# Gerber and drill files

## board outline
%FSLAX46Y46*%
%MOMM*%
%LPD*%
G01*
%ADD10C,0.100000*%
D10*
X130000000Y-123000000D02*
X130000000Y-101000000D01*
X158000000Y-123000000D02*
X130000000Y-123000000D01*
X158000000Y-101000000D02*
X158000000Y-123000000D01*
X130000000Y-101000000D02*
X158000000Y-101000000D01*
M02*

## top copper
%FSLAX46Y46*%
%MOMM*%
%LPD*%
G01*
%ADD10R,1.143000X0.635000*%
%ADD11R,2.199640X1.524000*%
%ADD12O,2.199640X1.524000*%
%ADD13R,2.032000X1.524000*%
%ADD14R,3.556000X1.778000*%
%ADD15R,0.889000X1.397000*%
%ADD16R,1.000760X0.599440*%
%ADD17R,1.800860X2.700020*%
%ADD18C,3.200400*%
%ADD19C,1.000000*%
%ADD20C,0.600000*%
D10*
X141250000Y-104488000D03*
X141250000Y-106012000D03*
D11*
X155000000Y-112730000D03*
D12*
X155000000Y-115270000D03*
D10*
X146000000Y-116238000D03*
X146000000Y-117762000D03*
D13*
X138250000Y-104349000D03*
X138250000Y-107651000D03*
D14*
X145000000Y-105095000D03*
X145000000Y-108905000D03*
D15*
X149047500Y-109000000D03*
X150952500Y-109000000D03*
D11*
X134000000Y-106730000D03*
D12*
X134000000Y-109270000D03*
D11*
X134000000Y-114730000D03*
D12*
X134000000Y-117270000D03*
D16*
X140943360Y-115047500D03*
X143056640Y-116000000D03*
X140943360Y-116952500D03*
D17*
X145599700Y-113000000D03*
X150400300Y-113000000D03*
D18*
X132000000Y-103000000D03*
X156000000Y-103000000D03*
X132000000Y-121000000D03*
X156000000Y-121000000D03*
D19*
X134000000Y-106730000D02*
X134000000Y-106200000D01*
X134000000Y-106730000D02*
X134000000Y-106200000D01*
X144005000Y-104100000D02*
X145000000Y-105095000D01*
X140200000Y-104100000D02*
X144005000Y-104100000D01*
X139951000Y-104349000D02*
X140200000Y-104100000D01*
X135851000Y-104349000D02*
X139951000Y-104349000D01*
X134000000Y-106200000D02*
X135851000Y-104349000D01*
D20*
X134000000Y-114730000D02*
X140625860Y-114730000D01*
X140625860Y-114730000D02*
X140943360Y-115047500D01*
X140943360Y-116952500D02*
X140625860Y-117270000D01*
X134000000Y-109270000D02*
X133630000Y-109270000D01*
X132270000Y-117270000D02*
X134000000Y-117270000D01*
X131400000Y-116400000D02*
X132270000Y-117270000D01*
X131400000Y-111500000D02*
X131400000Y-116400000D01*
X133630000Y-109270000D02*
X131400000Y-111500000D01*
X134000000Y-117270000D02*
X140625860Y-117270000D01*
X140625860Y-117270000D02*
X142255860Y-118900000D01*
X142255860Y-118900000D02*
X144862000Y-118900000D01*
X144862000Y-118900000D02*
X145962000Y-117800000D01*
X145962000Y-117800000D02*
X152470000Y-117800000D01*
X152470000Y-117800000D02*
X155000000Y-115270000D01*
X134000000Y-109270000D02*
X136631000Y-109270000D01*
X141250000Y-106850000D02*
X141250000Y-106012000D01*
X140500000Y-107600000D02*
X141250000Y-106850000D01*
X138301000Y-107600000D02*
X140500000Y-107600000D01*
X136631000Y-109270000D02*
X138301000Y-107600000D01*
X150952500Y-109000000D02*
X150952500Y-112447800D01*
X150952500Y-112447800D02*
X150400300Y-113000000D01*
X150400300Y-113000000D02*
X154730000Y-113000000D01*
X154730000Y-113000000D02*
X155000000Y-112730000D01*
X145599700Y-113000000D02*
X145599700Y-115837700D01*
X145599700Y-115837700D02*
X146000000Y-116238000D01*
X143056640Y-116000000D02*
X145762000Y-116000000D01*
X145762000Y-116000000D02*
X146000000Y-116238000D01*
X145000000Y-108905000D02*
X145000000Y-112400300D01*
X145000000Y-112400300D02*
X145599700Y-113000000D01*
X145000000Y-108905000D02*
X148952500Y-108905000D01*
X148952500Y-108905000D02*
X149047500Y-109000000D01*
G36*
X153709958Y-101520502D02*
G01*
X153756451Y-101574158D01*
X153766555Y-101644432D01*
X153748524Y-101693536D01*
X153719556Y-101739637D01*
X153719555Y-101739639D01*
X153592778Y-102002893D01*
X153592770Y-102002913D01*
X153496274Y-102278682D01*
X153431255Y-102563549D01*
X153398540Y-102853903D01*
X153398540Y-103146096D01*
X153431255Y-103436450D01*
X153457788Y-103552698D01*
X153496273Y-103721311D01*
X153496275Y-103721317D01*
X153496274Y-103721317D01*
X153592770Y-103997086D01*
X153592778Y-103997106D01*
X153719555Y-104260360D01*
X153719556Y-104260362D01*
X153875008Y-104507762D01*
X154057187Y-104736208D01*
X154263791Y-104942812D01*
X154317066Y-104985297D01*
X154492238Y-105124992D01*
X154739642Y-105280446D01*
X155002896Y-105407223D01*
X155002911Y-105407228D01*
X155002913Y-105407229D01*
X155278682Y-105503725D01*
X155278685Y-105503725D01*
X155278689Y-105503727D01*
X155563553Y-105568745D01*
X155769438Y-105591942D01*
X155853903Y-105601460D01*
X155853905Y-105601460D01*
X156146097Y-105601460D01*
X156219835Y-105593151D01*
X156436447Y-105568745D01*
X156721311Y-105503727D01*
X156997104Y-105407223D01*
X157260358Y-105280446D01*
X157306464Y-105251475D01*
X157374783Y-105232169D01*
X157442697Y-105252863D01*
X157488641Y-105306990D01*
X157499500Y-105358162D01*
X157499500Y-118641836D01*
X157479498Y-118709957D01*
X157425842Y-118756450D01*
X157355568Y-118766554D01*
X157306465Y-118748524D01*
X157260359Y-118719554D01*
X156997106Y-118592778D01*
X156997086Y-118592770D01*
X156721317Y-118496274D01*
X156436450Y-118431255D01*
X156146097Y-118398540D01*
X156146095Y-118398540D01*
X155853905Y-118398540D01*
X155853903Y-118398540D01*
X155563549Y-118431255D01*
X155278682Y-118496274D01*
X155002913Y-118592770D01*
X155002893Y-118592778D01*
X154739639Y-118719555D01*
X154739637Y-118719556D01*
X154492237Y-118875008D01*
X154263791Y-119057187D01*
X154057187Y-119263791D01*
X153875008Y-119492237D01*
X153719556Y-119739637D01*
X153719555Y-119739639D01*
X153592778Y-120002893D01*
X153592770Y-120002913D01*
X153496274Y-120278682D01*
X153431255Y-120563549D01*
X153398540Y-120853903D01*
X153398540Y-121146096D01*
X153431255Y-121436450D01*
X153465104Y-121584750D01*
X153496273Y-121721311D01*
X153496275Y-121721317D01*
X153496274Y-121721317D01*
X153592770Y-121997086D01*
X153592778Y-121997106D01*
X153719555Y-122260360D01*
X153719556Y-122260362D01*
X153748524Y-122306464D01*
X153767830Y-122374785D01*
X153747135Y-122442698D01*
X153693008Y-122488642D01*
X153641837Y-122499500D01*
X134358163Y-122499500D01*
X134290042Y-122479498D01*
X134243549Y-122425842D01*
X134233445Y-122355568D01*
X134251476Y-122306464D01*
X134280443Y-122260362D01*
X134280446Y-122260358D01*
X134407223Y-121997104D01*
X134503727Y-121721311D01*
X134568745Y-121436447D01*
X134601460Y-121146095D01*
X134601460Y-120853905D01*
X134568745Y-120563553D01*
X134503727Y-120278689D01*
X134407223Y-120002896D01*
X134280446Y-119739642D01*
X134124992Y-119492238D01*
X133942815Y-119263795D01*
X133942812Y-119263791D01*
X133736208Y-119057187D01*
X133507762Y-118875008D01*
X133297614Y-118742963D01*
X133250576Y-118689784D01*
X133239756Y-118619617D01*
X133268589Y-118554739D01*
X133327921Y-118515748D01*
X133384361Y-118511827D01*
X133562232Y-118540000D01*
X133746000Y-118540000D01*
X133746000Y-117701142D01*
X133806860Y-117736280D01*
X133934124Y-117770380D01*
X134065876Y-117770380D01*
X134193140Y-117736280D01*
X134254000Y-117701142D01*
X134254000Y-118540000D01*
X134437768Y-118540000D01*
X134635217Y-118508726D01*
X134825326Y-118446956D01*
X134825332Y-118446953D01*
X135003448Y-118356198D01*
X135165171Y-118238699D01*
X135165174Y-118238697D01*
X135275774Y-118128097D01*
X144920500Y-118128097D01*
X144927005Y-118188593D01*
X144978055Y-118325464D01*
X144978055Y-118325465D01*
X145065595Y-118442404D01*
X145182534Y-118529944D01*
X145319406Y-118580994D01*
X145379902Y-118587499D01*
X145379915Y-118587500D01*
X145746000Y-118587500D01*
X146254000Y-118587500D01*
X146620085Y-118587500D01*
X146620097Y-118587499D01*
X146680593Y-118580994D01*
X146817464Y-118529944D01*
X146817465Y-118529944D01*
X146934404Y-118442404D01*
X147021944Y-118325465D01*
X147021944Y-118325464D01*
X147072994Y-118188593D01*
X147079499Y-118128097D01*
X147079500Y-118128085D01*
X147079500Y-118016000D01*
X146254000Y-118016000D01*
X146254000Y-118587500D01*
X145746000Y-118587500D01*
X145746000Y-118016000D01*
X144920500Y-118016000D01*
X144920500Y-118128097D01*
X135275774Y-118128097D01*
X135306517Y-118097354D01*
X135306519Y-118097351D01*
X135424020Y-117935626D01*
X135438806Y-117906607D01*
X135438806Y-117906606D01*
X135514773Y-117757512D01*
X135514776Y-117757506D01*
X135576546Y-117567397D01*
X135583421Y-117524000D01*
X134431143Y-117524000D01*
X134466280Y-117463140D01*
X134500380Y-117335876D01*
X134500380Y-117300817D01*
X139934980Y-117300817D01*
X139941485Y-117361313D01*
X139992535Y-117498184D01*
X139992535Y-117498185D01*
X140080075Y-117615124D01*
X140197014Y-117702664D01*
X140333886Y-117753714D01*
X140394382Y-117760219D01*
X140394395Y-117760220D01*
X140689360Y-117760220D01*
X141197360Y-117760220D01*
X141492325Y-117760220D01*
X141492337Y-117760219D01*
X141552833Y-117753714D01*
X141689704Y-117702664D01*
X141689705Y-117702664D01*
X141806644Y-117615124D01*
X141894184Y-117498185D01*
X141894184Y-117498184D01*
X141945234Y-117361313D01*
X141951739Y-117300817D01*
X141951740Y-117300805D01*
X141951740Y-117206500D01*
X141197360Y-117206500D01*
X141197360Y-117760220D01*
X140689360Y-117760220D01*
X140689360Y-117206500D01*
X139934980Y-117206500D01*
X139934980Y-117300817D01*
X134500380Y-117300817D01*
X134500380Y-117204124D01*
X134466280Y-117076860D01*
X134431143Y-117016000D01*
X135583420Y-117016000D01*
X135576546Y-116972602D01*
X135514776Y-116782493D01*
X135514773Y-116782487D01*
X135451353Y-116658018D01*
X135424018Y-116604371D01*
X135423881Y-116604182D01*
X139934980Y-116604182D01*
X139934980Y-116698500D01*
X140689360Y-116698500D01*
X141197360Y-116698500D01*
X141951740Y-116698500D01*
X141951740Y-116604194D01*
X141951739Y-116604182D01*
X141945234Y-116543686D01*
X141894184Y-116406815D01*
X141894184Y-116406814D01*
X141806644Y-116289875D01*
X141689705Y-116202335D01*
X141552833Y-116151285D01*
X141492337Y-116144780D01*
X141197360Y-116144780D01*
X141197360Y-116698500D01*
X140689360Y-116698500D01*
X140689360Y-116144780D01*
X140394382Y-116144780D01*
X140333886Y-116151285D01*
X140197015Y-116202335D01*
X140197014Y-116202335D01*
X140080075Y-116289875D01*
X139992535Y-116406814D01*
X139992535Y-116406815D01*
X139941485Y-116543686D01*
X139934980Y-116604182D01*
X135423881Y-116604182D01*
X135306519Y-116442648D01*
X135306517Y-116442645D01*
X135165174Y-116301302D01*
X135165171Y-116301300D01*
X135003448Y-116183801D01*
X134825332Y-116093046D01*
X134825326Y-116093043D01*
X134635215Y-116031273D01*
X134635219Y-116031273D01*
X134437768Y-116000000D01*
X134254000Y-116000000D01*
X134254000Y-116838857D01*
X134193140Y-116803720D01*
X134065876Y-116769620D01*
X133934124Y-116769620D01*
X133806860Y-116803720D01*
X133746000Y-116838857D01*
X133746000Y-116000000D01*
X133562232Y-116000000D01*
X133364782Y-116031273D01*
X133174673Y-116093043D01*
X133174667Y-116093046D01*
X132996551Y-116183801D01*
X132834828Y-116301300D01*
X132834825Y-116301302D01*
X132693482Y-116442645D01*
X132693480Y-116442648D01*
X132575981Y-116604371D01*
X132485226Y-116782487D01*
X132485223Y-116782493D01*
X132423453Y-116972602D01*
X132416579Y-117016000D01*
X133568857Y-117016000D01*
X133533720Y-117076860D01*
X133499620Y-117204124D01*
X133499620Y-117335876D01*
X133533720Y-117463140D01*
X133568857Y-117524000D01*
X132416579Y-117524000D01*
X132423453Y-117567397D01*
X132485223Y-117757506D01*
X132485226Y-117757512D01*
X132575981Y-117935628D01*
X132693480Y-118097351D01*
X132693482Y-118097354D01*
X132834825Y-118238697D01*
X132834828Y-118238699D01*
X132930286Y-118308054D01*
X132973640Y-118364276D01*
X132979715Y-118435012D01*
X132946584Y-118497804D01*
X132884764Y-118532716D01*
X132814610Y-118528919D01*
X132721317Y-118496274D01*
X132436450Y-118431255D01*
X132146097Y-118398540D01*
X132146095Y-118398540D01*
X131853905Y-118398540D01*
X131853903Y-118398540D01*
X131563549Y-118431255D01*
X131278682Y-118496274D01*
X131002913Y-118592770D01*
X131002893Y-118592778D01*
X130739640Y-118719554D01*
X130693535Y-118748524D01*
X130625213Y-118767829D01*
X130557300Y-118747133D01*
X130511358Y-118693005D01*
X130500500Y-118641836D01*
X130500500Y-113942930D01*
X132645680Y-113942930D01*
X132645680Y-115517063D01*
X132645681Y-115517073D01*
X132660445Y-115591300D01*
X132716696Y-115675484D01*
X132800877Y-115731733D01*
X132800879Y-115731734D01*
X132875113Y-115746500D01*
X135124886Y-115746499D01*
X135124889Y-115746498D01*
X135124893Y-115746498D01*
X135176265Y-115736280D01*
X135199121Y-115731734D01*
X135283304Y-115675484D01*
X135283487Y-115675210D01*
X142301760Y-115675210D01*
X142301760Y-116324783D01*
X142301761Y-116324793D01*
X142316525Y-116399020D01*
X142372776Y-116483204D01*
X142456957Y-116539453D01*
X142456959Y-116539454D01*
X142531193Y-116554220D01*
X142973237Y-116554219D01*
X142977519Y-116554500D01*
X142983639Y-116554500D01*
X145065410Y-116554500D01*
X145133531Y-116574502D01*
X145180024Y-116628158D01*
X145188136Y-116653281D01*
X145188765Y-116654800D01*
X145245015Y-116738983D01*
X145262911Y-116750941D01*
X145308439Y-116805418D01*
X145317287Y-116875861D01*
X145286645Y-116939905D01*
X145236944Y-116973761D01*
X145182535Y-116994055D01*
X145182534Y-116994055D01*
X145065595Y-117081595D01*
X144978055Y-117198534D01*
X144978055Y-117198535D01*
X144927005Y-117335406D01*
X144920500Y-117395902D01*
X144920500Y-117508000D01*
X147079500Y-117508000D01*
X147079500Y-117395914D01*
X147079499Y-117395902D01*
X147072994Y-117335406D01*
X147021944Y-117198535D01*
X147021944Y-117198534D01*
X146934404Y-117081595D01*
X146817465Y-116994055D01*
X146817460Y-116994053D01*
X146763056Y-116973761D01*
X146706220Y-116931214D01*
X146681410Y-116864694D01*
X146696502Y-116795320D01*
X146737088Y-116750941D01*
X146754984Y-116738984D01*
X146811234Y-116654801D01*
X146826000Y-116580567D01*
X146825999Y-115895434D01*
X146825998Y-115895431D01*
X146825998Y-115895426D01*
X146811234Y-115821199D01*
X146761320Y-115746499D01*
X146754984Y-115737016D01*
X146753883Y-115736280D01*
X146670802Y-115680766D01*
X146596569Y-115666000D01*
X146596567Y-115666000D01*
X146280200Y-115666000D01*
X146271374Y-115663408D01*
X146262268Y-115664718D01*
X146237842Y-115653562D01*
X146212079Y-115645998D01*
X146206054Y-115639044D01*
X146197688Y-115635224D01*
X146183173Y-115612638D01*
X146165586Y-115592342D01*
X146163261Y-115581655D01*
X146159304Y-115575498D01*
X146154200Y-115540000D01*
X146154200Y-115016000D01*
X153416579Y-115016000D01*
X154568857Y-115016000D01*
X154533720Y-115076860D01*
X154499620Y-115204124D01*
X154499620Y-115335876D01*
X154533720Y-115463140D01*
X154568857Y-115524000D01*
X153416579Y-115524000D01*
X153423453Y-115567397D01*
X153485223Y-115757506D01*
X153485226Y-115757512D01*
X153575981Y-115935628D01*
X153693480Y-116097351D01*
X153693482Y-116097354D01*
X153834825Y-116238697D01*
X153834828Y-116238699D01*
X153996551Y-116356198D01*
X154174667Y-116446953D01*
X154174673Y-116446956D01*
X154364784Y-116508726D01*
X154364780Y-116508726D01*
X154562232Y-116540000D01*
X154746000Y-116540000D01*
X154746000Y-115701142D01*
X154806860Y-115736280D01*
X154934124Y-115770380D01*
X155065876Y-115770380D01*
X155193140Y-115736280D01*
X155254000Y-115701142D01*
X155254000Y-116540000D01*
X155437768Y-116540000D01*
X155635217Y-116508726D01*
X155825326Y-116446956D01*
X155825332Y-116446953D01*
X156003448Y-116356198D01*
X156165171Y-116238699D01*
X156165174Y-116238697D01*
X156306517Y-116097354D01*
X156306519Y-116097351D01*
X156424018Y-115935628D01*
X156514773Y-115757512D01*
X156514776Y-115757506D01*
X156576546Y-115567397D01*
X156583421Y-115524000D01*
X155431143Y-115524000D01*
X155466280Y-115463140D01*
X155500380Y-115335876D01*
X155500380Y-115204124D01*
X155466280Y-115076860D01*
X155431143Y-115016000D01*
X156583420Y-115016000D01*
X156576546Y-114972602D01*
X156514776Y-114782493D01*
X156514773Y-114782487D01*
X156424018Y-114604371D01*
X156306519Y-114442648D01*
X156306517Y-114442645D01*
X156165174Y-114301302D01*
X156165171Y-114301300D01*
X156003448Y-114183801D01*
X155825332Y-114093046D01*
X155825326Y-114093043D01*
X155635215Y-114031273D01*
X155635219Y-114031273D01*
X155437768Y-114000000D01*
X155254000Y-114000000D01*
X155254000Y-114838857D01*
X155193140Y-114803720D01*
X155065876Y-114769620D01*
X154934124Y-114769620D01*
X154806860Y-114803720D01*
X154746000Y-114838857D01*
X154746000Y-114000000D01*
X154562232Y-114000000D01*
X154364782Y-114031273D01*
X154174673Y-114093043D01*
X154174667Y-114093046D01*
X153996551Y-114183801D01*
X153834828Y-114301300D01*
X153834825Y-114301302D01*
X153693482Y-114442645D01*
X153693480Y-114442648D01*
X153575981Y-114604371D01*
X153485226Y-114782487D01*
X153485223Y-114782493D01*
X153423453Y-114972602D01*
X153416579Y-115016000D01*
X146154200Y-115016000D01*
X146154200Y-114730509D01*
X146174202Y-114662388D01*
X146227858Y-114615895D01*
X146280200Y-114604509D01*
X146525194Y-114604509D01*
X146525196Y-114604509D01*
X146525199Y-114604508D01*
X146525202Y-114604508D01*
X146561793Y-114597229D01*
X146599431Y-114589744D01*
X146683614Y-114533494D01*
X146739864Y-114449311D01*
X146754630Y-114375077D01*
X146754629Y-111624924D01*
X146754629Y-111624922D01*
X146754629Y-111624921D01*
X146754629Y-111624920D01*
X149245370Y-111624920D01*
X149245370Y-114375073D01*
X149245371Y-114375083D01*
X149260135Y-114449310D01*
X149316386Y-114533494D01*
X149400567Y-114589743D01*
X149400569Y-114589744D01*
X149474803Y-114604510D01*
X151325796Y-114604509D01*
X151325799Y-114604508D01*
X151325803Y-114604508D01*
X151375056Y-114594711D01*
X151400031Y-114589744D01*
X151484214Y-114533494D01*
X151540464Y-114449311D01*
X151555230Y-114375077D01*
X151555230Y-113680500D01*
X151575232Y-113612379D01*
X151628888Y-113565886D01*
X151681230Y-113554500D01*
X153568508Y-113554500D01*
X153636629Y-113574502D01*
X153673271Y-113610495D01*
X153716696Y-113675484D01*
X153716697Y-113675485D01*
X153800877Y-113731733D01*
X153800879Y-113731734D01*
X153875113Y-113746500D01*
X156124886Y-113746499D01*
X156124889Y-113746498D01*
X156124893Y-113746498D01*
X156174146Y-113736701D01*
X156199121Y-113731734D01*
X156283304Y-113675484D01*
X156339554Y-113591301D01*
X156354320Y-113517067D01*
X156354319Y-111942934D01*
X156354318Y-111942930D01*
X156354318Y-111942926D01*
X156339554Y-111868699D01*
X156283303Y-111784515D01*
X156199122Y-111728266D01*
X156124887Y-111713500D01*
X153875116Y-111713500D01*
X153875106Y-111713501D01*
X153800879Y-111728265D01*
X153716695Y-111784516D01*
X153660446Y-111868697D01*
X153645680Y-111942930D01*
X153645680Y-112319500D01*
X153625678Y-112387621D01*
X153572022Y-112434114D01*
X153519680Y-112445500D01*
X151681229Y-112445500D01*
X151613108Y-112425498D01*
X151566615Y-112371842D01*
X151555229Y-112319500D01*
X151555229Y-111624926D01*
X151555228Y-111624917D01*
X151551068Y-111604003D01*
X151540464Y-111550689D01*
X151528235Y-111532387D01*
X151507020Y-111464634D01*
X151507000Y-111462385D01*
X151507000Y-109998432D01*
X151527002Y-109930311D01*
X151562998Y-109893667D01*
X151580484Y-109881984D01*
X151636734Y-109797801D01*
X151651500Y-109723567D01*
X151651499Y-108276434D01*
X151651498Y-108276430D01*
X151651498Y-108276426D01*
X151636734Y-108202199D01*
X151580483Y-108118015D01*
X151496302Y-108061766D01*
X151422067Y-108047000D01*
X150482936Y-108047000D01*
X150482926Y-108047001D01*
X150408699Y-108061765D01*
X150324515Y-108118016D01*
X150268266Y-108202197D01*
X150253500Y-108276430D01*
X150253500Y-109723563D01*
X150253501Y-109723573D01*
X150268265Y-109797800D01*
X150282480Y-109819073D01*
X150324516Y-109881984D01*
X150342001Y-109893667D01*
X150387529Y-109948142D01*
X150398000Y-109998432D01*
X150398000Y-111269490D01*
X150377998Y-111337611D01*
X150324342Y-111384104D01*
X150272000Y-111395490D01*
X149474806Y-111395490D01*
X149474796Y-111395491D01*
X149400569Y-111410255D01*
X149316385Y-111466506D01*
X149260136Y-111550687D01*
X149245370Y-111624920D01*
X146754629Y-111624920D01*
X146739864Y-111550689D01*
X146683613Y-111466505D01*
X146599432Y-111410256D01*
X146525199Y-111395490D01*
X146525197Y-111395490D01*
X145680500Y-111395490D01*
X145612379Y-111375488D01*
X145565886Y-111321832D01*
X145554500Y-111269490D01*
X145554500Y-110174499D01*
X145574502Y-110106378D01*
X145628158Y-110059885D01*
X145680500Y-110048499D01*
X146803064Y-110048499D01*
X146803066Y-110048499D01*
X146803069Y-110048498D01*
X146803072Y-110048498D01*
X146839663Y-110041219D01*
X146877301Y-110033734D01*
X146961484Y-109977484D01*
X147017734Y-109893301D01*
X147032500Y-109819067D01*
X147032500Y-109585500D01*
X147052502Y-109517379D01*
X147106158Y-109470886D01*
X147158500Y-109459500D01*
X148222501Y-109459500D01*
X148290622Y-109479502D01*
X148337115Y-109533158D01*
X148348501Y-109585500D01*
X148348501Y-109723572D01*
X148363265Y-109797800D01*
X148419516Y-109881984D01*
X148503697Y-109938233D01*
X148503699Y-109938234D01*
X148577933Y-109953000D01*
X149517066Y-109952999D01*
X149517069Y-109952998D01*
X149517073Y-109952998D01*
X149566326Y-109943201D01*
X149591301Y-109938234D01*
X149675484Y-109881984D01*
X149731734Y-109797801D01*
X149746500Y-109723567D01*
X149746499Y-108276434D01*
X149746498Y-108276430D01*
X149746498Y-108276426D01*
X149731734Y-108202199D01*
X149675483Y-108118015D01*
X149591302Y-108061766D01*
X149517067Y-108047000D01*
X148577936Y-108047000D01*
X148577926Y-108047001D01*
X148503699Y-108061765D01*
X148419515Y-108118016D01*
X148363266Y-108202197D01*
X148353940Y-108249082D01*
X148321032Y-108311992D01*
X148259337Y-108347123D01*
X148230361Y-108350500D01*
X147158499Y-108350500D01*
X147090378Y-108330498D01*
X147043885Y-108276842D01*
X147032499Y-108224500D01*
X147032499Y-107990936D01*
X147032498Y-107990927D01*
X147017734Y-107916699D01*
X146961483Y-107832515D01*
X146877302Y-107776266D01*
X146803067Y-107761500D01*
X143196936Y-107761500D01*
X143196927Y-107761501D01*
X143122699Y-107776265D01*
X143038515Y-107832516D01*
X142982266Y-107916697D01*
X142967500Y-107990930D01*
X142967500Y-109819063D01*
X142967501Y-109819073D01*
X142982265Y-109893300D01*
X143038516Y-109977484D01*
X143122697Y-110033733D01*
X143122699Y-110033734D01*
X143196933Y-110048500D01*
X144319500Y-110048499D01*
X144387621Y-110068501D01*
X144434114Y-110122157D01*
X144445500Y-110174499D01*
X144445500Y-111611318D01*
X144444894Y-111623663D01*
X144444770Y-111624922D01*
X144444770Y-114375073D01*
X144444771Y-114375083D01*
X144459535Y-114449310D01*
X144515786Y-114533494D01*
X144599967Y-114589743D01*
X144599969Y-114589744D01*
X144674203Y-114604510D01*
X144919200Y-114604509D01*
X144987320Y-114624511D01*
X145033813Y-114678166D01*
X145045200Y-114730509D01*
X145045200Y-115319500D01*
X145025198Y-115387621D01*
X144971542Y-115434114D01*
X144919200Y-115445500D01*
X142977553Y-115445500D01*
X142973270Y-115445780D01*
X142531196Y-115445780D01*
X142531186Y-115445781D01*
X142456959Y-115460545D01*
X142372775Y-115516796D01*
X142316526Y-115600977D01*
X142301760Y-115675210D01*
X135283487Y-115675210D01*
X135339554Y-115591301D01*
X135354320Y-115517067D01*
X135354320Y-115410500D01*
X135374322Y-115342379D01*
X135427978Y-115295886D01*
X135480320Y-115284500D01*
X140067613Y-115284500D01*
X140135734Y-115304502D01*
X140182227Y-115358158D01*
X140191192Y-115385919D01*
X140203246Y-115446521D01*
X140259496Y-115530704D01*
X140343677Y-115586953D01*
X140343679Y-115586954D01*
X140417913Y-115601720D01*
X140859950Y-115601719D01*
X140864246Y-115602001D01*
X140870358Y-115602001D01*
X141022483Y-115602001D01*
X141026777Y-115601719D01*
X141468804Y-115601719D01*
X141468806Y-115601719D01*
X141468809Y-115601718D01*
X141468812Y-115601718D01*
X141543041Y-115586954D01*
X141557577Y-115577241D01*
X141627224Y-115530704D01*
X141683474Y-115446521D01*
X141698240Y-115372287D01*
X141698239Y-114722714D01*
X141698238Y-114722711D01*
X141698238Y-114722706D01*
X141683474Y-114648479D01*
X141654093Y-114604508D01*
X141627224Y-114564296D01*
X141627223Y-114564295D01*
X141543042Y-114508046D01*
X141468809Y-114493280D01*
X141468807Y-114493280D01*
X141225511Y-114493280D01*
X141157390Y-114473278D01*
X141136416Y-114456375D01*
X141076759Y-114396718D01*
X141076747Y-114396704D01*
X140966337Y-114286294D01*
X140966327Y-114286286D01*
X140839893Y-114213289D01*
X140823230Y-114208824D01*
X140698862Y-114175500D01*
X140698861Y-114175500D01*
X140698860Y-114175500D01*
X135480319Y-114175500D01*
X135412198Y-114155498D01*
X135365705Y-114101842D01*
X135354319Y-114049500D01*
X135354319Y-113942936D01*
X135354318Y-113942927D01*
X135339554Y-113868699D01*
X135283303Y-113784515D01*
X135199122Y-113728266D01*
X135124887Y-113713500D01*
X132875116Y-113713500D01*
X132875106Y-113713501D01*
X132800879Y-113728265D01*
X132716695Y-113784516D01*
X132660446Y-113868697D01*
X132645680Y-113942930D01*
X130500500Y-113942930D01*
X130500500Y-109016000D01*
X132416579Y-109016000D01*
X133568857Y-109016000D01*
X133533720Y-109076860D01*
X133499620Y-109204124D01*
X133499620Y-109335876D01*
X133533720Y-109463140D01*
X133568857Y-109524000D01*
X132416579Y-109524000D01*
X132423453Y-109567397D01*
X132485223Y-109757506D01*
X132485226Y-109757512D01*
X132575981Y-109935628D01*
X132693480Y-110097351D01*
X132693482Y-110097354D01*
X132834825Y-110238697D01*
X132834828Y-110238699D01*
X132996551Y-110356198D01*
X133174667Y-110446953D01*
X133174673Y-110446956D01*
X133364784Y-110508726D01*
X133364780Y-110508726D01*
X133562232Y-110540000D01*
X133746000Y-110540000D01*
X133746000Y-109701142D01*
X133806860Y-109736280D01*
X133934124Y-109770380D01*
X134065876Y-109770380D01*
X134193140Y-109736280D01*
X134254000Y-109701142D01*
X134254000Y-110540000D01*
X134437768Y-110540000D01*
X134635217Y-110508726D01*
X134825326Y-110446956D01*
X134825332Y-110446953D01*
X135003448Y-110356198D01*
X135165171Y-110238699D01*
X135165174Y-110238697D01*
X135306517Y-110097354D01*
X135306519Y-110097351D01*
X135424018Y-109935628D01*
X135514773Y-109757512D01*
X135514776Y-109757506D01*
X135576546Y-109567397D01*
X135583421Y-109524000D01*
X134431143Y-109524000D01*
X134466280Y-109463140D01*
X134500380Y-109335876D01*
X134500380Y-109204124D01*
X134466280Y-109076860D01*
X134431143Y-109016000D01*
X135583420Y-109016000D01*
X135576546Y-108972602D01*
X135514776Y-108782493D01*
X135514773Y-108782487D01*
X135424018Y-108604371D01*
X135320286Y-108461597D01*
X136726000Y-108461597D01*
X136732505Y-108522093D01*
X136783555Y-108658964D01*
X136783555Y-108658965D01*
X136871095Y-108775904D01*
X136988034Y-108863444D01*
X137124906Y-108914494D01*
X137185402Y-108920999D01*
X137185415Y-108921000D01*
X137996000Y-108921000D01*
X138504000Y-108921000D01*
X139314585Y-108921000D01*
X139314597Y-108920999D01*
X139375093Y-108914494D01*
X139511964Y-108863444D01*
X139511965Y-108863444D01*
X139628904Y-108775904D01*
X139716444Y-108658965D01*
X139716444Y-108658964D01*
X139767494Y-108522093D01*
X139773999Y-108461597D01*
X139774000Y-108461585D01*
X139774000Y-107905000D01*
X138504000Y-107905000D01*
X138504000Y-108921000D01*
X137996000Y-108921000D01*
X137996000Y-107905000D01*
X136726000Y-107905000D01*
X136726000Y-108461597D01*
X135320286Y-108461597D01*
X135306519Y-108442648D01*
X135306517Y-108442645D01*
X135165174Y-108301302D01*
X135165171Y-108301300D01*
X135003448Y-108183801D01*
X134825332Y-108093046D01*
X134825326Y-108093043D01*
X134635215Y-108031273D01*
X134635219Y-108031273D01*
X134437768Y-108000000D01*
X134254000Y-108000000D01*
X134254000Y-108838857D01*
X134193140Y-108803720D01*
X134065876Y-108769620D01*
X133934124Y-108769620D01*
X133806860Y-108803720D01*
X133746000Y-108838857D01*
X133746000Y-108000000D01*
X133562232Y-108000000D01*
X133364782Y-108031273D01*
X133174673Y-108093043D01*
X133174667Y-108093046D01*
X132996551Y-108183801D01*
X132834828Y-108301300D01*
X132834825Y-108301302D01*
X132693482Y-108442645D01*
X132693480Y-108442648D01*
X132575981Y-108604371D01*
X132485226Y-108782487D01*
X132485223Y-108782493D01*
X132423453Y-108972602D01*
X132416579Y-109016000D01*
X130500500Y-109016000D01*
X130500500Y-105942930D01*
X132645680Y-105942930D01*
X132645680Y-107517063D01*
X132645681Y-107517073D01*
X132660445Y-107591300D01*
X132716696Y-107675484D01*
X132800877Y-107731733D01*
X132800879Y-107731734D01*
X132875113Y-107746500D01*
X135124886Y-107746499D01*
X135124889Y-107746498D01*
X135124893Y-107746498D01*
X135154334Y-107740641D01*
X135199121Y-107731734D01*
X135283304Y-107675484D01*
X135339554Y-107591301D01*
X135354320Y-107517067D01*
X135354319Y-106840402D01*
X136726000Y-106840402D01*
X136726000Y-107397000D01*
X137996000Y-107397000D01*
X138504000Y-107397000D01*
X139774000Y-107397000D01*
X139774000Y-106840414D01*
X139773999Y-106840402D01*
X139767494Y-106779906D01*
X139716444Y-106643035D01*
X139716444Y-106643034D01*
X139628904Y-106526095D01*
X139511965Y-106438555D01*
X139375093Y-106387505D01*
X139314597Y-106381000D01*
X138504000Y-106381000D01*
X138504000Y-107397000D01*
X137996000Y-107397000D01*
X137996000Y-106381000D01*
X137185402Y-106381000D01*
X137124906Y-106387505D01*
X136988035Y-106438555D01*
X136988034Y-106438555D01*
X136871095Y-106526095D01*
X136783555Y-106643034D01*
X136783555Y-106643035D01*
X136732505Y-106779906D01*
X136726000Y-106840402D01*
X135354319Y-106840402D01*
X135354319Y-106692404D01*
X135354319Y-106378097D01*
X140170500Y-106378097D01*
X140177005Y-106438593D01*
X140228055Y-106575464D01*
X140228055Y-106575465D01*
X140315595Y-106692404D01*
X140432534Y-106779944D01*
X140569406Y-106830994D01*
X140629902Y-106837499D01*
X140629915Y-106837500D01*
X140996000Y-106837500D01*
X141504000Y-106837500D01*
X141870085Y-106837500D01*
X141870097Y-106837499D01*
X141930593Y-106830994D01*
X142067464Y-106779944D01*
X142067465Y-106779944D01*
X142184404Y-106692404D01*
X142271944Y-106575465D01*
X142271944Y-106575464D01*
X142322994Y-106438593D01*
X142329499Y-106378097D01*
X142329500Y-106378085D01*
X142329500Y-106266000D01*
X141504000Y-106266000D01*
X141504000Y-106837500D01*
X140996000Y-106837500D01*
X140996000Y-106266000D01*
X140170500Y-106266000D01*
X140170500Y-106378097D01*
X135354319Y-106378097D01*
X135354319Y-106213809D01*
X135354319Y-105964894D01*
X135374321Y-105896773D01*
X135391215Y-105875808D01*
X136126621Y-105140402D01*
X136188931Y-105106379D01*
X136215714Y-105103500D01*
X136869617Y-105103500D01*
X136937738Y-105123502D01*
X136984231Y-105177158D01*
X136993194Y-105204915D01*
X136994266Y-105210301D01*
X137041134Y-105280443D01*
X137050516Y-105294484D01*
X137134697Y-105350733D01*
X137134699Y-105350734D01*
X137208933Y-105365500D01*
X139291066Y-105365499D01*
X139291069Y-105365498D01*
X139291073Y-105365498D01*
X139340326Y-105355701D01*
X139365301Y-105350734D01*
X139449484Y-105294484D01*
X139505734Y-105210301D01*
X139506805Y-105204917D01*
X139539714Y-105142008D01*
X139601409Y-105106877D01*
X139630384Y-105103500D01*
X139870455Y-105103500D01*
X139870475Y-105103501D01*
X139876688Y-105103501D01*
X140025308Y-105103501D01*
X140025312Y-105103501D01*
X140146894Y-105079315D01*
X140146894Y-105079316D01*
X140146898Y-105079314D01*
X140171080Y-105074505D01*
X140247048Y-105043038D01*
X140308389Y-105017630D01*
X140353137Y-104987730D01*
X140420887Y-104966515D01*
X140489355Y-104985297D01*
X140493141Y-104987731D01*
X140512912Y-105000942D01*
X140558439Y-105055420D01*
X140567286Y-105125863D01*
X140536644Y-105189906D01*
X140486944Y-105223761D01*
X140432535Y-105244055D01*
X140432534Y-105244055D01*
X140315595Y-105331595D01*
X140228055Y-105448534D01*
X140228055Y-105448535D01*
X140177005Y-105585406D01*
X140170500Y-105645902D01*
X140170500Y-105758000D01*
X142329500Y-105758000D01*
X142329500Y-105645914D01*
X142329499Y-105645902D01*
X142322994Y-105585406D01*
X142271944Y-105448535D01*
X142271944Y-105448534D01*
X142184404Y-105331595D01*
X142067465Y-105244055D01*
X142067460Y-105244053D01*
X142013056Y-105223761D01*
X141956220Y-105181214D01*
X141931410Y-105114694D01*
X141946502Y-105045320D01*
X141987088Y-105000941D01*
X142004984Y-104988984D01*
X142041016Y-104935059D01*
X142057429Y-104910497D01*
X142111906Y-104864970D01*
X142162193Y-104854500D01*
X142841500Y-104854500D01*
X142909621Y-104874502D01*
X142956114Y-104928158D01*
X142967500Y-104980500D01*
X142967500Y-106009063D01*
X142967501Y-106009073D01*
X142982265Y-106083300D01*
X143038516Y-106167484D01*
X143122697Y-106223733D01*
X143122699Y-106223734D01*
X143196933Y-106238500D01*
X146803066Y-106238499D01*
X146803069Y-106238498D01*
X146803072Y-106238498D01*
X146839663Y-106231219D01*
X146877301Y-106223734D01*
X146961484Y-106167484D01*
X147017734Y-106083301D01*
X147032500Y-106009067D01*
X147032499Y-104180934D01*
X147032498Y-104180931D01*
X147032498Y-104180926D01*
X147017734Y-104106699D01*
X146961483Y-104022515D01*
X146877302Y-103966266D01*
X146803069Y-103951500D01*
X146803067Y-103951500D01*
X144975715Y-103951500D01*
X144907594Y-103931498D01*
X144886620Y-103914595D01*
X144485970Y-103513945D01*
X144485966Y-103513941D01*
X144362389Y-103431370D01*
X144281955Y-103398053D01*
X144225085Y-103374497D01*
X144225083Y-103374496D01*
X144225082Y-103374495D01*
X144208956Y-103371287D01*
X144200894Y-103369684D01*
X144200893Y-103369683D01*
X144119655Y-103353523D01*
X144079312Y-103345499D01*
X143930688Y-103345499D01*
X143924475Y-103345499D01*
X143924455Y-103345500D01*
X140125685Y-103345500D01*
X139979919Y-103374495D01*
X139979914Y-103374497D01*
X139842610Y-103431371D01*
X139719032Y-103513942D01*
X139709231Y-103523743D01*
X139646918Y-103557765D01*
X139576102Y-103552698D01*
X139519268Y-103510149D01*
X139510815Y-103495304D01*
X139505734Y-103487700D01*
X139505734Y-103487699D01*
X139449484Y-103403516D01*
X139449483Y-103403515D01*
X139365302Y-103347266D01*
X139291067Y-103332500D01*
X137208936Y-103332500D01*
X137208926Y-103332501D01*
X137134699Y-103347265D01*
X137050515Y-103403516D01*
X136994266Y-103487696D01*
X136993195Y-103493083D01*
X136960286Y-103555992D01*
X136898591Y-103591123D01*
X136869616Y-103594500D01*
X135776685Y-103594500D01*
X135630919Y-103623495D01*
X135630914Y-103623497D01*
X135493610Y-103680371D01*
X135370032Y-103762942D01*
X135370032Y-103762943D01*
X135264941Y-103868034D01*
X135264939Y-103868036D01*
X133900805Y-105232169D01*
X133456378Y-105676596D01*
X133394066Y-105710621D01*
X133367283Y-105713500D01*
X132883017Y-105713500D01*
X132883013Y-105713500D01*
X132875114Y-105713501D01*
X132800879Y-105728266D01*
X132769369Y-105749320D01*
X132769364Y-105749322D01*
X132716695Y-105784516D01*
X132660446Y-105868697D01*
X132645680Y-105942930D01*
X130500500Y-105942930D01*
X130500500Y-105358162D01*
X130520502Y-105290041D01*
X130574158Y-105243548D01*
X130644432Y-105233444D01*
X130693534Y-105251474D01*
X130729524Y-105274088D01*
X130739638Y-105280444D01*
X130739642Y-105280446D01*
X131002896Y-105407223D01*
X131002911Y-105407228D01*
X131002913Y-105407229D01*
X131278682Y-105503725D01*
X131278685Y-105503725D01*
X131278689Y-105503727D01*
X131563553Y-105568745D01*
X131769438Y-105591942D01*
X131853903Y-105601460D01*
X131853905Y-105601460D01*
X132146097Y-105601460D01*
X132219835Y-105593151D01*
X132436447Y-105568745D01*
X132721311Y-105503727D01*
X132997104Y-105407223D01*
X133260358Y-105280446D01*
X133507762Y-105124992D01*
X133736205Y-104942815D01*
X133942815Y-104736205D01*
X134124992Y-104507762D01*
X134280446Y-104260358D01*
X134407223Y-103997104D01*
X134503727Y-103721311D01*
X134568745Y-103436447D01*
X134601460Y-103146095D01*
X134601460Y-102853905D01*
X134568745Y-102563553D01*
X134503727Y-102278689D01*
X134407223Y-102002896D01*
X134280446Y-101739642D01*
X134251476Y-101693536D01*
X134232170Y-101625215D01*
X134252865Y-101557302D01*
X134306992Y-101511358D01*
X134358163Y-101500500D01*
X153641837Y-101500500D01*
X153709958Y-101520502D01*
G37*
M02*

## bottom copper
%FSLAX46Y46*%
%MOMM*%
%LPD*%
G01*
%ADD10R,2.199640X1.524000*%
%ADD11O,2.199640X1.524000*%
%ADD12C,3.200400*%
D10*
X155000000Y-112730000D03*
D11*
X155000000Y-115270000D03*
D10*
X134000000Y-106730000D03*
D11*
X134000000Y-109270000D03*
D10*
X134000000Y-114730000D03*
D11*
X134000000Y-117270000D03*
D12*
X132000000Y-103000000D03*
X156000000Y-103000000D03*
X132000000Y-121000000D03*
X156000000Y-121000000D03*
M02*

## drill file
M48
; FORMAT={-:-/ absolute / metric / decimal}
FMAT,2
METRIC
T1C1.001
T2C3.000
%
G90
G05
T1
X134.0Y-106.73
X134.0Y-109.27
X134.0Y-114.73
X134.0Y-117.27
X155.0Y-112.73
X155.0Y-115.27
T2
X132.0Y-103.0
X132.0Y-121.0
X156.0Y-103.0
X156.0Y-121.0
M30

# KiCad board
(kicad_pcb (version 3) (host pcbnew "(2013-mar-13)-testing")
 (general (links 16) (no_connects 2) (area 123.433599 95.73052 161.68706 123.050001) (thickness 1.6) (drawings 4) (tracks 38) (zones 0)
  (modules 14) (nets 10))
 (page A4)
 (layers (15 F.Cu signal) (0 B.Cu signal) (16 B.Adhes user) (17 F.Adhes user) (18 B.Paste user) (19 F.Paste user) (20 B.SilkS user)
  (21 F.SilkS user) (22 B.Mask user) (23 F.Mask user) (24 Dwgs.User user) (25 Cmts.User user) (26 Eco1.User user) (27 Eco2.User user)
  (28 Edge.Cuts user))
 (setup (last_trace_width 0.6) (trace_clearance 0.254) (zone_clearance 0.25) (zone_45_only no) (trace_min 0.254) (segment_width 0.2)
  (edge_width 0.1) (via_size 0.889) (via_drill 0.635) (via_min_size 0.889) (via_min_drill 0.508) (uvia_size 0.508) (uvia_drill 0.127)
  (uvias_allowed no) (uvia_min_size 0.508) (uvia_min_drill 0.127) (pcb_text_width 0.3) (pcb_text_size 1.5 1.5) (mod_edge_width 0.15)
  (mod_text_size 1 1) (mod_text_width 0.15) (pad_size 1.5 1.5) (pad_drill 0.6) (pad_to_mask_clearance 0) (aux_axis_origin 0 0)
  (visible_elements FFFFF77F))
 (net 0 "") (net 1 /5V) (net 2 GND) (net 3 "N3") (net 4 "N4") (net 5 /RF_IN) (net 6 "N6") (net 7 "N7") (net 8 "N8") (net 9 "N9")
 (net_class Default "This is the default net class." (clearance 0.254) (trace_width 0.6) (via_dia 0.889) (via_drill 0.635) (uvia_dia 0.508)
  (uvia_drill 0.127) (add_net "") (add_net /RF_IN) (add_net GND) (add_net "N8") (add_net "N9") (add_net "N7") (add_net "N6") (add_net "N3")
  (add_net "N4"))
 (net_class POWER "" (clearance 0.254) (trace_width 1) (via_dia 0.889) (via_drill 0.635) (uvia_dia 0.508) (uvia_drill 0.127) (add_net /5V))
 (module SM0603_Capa (layer F.Cu) (at 141.25 105.25 270)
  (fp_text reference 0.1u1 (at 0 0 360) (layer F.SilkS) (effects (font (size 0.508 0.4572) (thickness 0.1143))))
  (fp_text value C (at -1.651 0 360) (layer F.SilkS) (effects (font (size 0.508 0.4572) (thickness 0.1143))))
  (pad 1 smd rect (at -0.762 0 270) (size 0.635 1.143) (layers F.Cu F.Paste F.Mask) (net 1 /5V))
  (pad 2 smd rect (at 0.762 0 270) (size 0.635 1.143) (layers F.Cu F.Paste F.Mask) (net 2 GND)))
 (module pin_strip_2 (layer F.Cu) (at 155 114 270)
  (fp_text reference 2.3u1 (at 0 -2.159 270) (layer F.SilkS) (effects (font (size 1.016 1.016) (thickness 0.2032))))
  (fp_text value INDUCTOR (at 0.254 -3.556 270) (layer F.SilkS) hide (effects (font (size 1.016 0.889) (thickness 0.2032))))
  (pad 1 thru_hole rect (at -1.27 0 270) (size 1.524 2.19964) (drill 1.00076) (layers *.Cu *.Mask F.SilkS) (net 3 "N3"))
  (pad 2 thru_hole oval (at 1.27 0 270) (size 1.524 2.19964) (drill 1.00076) (layers *.Cu *.Mask F.SilkS) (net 2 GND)))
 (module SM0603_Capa (layer F.Cu) (at 146 117 270)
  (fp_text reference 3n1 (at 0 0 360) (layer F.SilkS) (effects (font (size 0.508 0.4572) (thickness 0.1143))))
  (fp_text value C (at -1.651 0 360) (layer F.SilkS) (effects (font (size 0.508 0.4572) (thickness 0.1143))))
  (pad 1 smd rect (at -0.762 0 270) (size 0.635 1.143) (layers F.Cu F.Paste F.Mask) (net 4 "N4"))
  (pad 2 smd rect (at 0.762 0 270) (size 0.635 1.143) (layers F.Cu F.Paste F.Mask) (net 2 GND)))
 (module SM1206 (layer F.Cu) (at 138.25 106 270)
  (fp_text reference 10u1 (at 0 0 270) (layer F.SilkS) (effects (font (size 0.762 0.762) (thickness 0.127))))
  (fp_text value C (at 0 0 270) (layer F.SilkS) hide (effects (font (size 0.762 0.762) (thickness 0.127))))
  (pad 1 smd rect (at -1.651 0 270) (size 1.524 2.032) (layers F.Cu F.Paste F.Mask) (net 1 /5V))
  (pad 2 smd rect (at 1.651 0 270) (size 1.524 2.032) (layers F.Cu F.Paste F.Mask) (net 2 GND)))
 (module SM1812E (layer F.Cu) (at 145 107 270)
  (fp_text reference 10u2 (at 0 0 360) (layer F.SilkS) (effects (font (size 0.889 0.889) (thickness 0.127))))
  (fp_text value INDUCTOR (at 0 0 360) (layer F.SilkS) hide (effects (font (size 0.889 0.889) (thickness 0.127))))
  (pad 1 smd rect (at -1.905 0 270) (size 1.778 3.556) (layers F.Cu F.Paste F.Mask) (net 1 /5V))
  (pad 2 smd rect (at 1.905 0 270) (size 1.778 3.556) (layers F.Cu F.Paste F.Mask) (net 4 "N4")))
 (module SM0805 (layer F.Cu) (at 150 109)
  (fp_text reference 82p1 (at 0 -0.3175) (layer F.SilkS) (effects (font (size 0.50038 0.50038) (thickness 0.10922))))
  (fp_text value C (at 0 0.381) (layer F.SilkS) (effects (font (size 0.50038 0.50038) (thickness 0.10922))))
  (pad 1 smd rect (at -0.9525 0) (size 0.889 1.397) (layers F.Cu F.Paste F.Mask) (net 4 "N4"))
  (pad 2 smd rect (at 0.9525 0) (size 0.889 1.397) (layers F.Cu F.Paste F.Mask) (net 3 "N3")))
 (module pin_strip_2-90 (layer F.Cu) (at 134 108 270)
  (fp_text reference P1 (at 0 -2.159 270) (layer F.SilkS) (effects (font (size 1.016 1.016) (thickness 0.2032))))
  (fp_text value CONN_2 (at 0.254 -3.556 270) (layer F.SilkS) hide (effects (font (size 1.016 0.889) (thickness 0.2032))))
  (pad 1 thru_hole rect (at -1.27 0 270) (size 1.524 2.19964) (drill 1.00076) (layers *.Cu *.Mask F.SilkS) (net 1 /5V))
  (pad 2 thru_hole oval (at 1.27 0 270) (size 1.524 2.19964) (drill 1.00076) (layers *.Cu *.Mask F.SilkS) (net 2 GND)))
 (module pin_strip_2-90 (layer F.Cu) (at 134 116 270)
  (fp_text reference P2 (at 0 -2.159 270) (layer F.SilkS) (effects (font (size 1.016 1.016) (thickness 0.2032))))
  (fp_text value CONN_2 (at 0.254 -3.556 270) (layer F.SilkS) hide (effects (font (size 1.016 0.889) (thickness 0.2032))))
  (pad 1 thru_hole rect (at -1.27 0 270) (size 1.524 2.19964) (drill 1.00076) (layers *.Cu *.Mask F.SilkS) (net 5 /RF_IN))
  (pad 2 thru_hole oval (at 1.27 0 270) (size 1.524 2.19964) (drill 1.00076) (layers *.Cu *.Mask F.SilkS) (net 2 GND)))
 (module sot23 (layer F.Cu) (at 142 116 270)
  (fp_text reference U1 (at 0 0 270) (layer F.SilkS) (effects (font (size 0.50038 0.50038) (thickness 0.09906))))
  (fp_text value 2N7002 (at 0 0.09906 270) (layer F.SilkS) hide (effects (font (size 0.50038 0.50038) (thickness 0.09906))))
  (pad 1 smd rect (at -0.9525 1.05664 270) (size 0.59944 1.00076) (layers F.Cu F.Paste F.Mask) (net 5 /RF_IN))
  (pad 2 smd rect (at 0 -1.05664 270) (size 0.59944 1.00076) (layers F.Cu F.Paste F.Mask) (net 4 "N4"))
  (pad 3 smd rect (at 0.9525 1.05664 270) (size 0.59944 1.00076) (layers F.Cu F.Paste F.Mask) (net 2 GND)))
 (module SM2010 (layer F.Cu) (at 148 113)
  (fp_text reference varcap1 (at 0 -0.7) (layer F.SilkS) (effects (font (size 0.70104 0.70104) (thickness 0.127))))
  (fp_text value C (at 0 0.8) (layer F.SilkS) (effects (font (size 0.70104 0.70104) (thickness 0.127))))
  (pad 1 smd rect (at -2.4003 0) (size 1.80086 2.70002) (layers F.Cu F.Paste F.Mask) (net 4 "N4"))
  (pad 2 smd rect (at 2.4003 0) (size 1.80086 2.70002) (layers F.Cu F.Paste F.Mask) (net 3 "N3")))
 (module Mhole (layer F.Cu) (at 132 103)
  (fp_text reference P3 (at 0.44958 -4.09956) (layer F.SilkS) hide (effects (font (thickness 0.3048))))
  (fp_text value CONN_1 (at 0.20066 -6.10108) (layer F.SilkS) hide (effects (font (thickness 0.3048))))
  (pad 1 thru_hole circle (at 0 0) (size 3.2004 3.2004) (drill 2.99974) (layers *.Cu *.Mask F.SilkS) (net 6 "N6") (clearance 1.00076)))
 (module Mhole (layer F.Cu) (at 156 103)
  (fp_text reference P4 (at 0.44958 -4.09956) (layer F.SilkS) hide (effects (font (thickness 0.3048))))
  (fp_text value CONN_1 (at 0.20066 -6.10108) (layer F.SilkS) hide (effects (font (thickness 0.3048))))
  (pad 1 thru_hole circle (at 0 0) (size 3.2004 3.2004) (drill 2.99974) (layers *.Cu *.Mask F.SilkS) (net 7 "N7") (clearance 1.00076)))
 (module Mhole (layer F.Cu) (at 132 121)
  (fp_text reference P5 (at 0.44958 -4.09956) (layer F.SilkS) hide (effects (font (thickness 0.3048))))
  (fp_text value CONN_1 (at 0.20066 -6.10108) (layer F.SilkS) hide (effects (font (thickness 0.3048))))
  (pad 1 thru_hole circle (at 0 0) (size 3.2004 3.2004) (drill 2.99974) (layers *.Cu *.Mask F.SilkS) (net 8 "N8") (clearance 1.00076)))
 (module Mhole (layer F.Cu) (at 156 121)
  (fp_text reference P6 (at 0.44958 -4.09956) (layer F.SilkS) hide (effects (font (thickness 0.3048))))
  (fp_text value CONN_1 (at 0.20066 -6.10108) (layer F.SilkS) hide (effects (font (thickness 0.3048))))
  (pad 1 thru_hole circle (at 0 0) (size 3.2004 3.2004) (drill 2.99974) (layers *.Cu *.Mask F.SilkS) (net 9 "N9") (clearance 1.00076)))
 (gr_line (start 130 123) (end 130 101) (angle 90) (layer Edge.Cuts) (width 0.1))
 (gr_line (start 158 123) (end 130 123) (angle 90) (layer Edge.Cuts) (width 0.1))
 (gr_line (start 158 101) (end 158 123) (angle 90) (layer Edge.Cuts) (width 0.1))
 (gr_line (start 130 101) (end 158 101) (angle 90) (layer Edge.Cuts) (width 0.1))
 (segment (start 134 106.73) (end 134 106.2) (width 1) (layer F.Cu) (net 1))
 (segment (start 134 106.73) (end 134 106.2) (width 1) (layer F.Cu) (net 1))
 (segment (start 144.005 104.1) (end 145 105.095) (width 1) (layer F.Cu) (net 1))
 (segment (start 140.2 104.1) (end 144.005 104.1) (width 1) (layer F.Cu) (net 1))
 (segment (start 139.951 104.349) (end 140.2 104.1) (width 1) (layer F.Cu) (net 1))
 (segment (start 135.851 104.349) (end 139.951 104.349) (width 1) (layer F.Cu) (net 1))
 (segment (start 134 106.2) (end 135.851 104.349) (width 1) (layer F.Cu) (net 1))
 (segment (start 134 114.73) (end 140.62586 114.73) (width 0.6) (layer F.Cu) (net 5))
 (segment (start 140.62586 114.73) (end 140.94336 115.0475) (width 0.6) (layer F.Cu) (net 5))
 (segment (start 140.94336 116.9525) (end 140.62586 117.27) (width 0.6) (layer F.Cu) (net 2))
 (segment (start 134 109.27) (end 133.63 109.27) (width 0.6) (layer F.Cu) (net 2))
 (segment (start 132.27 117.27) (end 134 117.27) (width 0.6) (layer F.Cu) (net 2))
 (segment (start 131.4 116.4) (end 132.27 117.27) (width 0.6) (layer F.Cu) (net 2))
 (segment (start 131.4 111.5) (end 131.4 116.4) (width 0.6) (layer F.Cu) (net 2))
 (segment (start 133.63 109.27) (end 131.4 111.5) (width 0.6) (layer F.Cu) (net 2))
 (segment (start 134 117.27) (end 140.62586 117.27) (width 0.6) (layer F.Cu) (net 2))
 (segment (start 140.62586 117.27) (end 142.25586 118.9) (width 0.6) (layer F.Cu) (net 2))
 (segment (start 142.25586 118.9) (end 144.862 118.9) (width 0.6) (layer F.Cu) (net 2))
 (segment (start 144.862 118.9) (end 145.962 117.8) (width 0.6) (layer F.Cu) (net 2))
 (segment (start 145.962 117.8) (end 152.47 117.8) (width 0.6) (layer F.Cu) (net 2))
 (segment (start 152.47 117.8) (end 155 115.27) (width 0.6) (layer F.Cu) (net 2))
 (segment (start 134 109.27) (end 136.631 109.27) (width 0.6) (layer F.Cu) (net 2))
 (segment (start 141.25 106.85) (end 141.25 106.012) (width 0.6) (layer F.Cu) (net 2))
 (segment (start 140.5 107.6) (end 141.25 106.85) (width 0.6) (layer F.Cu) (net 2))
 (segment (start 138.301 107.6) (end 140.5 107.6) (width 0.6) (layer F.Cu) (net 2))
 (segment (start 136.631 109.27) (end 138.301 107.6) (width 0.6) (layer F.Cu) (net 2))
 (segment (start 150.9525 109) (end 150.9525 112.4478) (width 0.6) (layer F.Cu) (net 3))
 (segment (start 150.9525 112.4478) (end 150.4003 113) (width 0.6) (layer F.Cu) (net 3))
 (segment (start 150.4003 113) (end 154.73 113) (width 0.6) (layer F.Cu) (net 3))
 (segment (start 154.73 113) (end 155 112.73) (width 0.6) (layer F.Cu) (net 3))
 (segment (start 145.5997 113) (end 145.5997 115.8377) (width 0.6) (layer F.Cu) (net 4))
 (segment (start 145.5997 115.8377) (end 146 116.238) (width 0.6) (layer F.Cu) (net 4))
 (segment (start 143.05664 116) (end 145.762 116) (width 0.6) (layer F.Cu) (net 4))
 (segment (start 145.762 116) (end 146 116.238) (width 0.6) (layer F.Cu) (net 4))
 (segment (start 145 108.905) (end 145 112.4003) (width 0.6) (layer F.Cu) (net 4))
 (segment (start 145 112.4003) (end 145.5997 113) (width 0.6) (layer F.Cu) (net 4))
 (segment (start 145 108.905) (end 148.9525 108.905) (width 0.6) (layer F.Cu) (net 4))
 (segment (start 148.9525 108.905) (end 149.0475 109) (width 0.6) (layer F.Cu) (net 4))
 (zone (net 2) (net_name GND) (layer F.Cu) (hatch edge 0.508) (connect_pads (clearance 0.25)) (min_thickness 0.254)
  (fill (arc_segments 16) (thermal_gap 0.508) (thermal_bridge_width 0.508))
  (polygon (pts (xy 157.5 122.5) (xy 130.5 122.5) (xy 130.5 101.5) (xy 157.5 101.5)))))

